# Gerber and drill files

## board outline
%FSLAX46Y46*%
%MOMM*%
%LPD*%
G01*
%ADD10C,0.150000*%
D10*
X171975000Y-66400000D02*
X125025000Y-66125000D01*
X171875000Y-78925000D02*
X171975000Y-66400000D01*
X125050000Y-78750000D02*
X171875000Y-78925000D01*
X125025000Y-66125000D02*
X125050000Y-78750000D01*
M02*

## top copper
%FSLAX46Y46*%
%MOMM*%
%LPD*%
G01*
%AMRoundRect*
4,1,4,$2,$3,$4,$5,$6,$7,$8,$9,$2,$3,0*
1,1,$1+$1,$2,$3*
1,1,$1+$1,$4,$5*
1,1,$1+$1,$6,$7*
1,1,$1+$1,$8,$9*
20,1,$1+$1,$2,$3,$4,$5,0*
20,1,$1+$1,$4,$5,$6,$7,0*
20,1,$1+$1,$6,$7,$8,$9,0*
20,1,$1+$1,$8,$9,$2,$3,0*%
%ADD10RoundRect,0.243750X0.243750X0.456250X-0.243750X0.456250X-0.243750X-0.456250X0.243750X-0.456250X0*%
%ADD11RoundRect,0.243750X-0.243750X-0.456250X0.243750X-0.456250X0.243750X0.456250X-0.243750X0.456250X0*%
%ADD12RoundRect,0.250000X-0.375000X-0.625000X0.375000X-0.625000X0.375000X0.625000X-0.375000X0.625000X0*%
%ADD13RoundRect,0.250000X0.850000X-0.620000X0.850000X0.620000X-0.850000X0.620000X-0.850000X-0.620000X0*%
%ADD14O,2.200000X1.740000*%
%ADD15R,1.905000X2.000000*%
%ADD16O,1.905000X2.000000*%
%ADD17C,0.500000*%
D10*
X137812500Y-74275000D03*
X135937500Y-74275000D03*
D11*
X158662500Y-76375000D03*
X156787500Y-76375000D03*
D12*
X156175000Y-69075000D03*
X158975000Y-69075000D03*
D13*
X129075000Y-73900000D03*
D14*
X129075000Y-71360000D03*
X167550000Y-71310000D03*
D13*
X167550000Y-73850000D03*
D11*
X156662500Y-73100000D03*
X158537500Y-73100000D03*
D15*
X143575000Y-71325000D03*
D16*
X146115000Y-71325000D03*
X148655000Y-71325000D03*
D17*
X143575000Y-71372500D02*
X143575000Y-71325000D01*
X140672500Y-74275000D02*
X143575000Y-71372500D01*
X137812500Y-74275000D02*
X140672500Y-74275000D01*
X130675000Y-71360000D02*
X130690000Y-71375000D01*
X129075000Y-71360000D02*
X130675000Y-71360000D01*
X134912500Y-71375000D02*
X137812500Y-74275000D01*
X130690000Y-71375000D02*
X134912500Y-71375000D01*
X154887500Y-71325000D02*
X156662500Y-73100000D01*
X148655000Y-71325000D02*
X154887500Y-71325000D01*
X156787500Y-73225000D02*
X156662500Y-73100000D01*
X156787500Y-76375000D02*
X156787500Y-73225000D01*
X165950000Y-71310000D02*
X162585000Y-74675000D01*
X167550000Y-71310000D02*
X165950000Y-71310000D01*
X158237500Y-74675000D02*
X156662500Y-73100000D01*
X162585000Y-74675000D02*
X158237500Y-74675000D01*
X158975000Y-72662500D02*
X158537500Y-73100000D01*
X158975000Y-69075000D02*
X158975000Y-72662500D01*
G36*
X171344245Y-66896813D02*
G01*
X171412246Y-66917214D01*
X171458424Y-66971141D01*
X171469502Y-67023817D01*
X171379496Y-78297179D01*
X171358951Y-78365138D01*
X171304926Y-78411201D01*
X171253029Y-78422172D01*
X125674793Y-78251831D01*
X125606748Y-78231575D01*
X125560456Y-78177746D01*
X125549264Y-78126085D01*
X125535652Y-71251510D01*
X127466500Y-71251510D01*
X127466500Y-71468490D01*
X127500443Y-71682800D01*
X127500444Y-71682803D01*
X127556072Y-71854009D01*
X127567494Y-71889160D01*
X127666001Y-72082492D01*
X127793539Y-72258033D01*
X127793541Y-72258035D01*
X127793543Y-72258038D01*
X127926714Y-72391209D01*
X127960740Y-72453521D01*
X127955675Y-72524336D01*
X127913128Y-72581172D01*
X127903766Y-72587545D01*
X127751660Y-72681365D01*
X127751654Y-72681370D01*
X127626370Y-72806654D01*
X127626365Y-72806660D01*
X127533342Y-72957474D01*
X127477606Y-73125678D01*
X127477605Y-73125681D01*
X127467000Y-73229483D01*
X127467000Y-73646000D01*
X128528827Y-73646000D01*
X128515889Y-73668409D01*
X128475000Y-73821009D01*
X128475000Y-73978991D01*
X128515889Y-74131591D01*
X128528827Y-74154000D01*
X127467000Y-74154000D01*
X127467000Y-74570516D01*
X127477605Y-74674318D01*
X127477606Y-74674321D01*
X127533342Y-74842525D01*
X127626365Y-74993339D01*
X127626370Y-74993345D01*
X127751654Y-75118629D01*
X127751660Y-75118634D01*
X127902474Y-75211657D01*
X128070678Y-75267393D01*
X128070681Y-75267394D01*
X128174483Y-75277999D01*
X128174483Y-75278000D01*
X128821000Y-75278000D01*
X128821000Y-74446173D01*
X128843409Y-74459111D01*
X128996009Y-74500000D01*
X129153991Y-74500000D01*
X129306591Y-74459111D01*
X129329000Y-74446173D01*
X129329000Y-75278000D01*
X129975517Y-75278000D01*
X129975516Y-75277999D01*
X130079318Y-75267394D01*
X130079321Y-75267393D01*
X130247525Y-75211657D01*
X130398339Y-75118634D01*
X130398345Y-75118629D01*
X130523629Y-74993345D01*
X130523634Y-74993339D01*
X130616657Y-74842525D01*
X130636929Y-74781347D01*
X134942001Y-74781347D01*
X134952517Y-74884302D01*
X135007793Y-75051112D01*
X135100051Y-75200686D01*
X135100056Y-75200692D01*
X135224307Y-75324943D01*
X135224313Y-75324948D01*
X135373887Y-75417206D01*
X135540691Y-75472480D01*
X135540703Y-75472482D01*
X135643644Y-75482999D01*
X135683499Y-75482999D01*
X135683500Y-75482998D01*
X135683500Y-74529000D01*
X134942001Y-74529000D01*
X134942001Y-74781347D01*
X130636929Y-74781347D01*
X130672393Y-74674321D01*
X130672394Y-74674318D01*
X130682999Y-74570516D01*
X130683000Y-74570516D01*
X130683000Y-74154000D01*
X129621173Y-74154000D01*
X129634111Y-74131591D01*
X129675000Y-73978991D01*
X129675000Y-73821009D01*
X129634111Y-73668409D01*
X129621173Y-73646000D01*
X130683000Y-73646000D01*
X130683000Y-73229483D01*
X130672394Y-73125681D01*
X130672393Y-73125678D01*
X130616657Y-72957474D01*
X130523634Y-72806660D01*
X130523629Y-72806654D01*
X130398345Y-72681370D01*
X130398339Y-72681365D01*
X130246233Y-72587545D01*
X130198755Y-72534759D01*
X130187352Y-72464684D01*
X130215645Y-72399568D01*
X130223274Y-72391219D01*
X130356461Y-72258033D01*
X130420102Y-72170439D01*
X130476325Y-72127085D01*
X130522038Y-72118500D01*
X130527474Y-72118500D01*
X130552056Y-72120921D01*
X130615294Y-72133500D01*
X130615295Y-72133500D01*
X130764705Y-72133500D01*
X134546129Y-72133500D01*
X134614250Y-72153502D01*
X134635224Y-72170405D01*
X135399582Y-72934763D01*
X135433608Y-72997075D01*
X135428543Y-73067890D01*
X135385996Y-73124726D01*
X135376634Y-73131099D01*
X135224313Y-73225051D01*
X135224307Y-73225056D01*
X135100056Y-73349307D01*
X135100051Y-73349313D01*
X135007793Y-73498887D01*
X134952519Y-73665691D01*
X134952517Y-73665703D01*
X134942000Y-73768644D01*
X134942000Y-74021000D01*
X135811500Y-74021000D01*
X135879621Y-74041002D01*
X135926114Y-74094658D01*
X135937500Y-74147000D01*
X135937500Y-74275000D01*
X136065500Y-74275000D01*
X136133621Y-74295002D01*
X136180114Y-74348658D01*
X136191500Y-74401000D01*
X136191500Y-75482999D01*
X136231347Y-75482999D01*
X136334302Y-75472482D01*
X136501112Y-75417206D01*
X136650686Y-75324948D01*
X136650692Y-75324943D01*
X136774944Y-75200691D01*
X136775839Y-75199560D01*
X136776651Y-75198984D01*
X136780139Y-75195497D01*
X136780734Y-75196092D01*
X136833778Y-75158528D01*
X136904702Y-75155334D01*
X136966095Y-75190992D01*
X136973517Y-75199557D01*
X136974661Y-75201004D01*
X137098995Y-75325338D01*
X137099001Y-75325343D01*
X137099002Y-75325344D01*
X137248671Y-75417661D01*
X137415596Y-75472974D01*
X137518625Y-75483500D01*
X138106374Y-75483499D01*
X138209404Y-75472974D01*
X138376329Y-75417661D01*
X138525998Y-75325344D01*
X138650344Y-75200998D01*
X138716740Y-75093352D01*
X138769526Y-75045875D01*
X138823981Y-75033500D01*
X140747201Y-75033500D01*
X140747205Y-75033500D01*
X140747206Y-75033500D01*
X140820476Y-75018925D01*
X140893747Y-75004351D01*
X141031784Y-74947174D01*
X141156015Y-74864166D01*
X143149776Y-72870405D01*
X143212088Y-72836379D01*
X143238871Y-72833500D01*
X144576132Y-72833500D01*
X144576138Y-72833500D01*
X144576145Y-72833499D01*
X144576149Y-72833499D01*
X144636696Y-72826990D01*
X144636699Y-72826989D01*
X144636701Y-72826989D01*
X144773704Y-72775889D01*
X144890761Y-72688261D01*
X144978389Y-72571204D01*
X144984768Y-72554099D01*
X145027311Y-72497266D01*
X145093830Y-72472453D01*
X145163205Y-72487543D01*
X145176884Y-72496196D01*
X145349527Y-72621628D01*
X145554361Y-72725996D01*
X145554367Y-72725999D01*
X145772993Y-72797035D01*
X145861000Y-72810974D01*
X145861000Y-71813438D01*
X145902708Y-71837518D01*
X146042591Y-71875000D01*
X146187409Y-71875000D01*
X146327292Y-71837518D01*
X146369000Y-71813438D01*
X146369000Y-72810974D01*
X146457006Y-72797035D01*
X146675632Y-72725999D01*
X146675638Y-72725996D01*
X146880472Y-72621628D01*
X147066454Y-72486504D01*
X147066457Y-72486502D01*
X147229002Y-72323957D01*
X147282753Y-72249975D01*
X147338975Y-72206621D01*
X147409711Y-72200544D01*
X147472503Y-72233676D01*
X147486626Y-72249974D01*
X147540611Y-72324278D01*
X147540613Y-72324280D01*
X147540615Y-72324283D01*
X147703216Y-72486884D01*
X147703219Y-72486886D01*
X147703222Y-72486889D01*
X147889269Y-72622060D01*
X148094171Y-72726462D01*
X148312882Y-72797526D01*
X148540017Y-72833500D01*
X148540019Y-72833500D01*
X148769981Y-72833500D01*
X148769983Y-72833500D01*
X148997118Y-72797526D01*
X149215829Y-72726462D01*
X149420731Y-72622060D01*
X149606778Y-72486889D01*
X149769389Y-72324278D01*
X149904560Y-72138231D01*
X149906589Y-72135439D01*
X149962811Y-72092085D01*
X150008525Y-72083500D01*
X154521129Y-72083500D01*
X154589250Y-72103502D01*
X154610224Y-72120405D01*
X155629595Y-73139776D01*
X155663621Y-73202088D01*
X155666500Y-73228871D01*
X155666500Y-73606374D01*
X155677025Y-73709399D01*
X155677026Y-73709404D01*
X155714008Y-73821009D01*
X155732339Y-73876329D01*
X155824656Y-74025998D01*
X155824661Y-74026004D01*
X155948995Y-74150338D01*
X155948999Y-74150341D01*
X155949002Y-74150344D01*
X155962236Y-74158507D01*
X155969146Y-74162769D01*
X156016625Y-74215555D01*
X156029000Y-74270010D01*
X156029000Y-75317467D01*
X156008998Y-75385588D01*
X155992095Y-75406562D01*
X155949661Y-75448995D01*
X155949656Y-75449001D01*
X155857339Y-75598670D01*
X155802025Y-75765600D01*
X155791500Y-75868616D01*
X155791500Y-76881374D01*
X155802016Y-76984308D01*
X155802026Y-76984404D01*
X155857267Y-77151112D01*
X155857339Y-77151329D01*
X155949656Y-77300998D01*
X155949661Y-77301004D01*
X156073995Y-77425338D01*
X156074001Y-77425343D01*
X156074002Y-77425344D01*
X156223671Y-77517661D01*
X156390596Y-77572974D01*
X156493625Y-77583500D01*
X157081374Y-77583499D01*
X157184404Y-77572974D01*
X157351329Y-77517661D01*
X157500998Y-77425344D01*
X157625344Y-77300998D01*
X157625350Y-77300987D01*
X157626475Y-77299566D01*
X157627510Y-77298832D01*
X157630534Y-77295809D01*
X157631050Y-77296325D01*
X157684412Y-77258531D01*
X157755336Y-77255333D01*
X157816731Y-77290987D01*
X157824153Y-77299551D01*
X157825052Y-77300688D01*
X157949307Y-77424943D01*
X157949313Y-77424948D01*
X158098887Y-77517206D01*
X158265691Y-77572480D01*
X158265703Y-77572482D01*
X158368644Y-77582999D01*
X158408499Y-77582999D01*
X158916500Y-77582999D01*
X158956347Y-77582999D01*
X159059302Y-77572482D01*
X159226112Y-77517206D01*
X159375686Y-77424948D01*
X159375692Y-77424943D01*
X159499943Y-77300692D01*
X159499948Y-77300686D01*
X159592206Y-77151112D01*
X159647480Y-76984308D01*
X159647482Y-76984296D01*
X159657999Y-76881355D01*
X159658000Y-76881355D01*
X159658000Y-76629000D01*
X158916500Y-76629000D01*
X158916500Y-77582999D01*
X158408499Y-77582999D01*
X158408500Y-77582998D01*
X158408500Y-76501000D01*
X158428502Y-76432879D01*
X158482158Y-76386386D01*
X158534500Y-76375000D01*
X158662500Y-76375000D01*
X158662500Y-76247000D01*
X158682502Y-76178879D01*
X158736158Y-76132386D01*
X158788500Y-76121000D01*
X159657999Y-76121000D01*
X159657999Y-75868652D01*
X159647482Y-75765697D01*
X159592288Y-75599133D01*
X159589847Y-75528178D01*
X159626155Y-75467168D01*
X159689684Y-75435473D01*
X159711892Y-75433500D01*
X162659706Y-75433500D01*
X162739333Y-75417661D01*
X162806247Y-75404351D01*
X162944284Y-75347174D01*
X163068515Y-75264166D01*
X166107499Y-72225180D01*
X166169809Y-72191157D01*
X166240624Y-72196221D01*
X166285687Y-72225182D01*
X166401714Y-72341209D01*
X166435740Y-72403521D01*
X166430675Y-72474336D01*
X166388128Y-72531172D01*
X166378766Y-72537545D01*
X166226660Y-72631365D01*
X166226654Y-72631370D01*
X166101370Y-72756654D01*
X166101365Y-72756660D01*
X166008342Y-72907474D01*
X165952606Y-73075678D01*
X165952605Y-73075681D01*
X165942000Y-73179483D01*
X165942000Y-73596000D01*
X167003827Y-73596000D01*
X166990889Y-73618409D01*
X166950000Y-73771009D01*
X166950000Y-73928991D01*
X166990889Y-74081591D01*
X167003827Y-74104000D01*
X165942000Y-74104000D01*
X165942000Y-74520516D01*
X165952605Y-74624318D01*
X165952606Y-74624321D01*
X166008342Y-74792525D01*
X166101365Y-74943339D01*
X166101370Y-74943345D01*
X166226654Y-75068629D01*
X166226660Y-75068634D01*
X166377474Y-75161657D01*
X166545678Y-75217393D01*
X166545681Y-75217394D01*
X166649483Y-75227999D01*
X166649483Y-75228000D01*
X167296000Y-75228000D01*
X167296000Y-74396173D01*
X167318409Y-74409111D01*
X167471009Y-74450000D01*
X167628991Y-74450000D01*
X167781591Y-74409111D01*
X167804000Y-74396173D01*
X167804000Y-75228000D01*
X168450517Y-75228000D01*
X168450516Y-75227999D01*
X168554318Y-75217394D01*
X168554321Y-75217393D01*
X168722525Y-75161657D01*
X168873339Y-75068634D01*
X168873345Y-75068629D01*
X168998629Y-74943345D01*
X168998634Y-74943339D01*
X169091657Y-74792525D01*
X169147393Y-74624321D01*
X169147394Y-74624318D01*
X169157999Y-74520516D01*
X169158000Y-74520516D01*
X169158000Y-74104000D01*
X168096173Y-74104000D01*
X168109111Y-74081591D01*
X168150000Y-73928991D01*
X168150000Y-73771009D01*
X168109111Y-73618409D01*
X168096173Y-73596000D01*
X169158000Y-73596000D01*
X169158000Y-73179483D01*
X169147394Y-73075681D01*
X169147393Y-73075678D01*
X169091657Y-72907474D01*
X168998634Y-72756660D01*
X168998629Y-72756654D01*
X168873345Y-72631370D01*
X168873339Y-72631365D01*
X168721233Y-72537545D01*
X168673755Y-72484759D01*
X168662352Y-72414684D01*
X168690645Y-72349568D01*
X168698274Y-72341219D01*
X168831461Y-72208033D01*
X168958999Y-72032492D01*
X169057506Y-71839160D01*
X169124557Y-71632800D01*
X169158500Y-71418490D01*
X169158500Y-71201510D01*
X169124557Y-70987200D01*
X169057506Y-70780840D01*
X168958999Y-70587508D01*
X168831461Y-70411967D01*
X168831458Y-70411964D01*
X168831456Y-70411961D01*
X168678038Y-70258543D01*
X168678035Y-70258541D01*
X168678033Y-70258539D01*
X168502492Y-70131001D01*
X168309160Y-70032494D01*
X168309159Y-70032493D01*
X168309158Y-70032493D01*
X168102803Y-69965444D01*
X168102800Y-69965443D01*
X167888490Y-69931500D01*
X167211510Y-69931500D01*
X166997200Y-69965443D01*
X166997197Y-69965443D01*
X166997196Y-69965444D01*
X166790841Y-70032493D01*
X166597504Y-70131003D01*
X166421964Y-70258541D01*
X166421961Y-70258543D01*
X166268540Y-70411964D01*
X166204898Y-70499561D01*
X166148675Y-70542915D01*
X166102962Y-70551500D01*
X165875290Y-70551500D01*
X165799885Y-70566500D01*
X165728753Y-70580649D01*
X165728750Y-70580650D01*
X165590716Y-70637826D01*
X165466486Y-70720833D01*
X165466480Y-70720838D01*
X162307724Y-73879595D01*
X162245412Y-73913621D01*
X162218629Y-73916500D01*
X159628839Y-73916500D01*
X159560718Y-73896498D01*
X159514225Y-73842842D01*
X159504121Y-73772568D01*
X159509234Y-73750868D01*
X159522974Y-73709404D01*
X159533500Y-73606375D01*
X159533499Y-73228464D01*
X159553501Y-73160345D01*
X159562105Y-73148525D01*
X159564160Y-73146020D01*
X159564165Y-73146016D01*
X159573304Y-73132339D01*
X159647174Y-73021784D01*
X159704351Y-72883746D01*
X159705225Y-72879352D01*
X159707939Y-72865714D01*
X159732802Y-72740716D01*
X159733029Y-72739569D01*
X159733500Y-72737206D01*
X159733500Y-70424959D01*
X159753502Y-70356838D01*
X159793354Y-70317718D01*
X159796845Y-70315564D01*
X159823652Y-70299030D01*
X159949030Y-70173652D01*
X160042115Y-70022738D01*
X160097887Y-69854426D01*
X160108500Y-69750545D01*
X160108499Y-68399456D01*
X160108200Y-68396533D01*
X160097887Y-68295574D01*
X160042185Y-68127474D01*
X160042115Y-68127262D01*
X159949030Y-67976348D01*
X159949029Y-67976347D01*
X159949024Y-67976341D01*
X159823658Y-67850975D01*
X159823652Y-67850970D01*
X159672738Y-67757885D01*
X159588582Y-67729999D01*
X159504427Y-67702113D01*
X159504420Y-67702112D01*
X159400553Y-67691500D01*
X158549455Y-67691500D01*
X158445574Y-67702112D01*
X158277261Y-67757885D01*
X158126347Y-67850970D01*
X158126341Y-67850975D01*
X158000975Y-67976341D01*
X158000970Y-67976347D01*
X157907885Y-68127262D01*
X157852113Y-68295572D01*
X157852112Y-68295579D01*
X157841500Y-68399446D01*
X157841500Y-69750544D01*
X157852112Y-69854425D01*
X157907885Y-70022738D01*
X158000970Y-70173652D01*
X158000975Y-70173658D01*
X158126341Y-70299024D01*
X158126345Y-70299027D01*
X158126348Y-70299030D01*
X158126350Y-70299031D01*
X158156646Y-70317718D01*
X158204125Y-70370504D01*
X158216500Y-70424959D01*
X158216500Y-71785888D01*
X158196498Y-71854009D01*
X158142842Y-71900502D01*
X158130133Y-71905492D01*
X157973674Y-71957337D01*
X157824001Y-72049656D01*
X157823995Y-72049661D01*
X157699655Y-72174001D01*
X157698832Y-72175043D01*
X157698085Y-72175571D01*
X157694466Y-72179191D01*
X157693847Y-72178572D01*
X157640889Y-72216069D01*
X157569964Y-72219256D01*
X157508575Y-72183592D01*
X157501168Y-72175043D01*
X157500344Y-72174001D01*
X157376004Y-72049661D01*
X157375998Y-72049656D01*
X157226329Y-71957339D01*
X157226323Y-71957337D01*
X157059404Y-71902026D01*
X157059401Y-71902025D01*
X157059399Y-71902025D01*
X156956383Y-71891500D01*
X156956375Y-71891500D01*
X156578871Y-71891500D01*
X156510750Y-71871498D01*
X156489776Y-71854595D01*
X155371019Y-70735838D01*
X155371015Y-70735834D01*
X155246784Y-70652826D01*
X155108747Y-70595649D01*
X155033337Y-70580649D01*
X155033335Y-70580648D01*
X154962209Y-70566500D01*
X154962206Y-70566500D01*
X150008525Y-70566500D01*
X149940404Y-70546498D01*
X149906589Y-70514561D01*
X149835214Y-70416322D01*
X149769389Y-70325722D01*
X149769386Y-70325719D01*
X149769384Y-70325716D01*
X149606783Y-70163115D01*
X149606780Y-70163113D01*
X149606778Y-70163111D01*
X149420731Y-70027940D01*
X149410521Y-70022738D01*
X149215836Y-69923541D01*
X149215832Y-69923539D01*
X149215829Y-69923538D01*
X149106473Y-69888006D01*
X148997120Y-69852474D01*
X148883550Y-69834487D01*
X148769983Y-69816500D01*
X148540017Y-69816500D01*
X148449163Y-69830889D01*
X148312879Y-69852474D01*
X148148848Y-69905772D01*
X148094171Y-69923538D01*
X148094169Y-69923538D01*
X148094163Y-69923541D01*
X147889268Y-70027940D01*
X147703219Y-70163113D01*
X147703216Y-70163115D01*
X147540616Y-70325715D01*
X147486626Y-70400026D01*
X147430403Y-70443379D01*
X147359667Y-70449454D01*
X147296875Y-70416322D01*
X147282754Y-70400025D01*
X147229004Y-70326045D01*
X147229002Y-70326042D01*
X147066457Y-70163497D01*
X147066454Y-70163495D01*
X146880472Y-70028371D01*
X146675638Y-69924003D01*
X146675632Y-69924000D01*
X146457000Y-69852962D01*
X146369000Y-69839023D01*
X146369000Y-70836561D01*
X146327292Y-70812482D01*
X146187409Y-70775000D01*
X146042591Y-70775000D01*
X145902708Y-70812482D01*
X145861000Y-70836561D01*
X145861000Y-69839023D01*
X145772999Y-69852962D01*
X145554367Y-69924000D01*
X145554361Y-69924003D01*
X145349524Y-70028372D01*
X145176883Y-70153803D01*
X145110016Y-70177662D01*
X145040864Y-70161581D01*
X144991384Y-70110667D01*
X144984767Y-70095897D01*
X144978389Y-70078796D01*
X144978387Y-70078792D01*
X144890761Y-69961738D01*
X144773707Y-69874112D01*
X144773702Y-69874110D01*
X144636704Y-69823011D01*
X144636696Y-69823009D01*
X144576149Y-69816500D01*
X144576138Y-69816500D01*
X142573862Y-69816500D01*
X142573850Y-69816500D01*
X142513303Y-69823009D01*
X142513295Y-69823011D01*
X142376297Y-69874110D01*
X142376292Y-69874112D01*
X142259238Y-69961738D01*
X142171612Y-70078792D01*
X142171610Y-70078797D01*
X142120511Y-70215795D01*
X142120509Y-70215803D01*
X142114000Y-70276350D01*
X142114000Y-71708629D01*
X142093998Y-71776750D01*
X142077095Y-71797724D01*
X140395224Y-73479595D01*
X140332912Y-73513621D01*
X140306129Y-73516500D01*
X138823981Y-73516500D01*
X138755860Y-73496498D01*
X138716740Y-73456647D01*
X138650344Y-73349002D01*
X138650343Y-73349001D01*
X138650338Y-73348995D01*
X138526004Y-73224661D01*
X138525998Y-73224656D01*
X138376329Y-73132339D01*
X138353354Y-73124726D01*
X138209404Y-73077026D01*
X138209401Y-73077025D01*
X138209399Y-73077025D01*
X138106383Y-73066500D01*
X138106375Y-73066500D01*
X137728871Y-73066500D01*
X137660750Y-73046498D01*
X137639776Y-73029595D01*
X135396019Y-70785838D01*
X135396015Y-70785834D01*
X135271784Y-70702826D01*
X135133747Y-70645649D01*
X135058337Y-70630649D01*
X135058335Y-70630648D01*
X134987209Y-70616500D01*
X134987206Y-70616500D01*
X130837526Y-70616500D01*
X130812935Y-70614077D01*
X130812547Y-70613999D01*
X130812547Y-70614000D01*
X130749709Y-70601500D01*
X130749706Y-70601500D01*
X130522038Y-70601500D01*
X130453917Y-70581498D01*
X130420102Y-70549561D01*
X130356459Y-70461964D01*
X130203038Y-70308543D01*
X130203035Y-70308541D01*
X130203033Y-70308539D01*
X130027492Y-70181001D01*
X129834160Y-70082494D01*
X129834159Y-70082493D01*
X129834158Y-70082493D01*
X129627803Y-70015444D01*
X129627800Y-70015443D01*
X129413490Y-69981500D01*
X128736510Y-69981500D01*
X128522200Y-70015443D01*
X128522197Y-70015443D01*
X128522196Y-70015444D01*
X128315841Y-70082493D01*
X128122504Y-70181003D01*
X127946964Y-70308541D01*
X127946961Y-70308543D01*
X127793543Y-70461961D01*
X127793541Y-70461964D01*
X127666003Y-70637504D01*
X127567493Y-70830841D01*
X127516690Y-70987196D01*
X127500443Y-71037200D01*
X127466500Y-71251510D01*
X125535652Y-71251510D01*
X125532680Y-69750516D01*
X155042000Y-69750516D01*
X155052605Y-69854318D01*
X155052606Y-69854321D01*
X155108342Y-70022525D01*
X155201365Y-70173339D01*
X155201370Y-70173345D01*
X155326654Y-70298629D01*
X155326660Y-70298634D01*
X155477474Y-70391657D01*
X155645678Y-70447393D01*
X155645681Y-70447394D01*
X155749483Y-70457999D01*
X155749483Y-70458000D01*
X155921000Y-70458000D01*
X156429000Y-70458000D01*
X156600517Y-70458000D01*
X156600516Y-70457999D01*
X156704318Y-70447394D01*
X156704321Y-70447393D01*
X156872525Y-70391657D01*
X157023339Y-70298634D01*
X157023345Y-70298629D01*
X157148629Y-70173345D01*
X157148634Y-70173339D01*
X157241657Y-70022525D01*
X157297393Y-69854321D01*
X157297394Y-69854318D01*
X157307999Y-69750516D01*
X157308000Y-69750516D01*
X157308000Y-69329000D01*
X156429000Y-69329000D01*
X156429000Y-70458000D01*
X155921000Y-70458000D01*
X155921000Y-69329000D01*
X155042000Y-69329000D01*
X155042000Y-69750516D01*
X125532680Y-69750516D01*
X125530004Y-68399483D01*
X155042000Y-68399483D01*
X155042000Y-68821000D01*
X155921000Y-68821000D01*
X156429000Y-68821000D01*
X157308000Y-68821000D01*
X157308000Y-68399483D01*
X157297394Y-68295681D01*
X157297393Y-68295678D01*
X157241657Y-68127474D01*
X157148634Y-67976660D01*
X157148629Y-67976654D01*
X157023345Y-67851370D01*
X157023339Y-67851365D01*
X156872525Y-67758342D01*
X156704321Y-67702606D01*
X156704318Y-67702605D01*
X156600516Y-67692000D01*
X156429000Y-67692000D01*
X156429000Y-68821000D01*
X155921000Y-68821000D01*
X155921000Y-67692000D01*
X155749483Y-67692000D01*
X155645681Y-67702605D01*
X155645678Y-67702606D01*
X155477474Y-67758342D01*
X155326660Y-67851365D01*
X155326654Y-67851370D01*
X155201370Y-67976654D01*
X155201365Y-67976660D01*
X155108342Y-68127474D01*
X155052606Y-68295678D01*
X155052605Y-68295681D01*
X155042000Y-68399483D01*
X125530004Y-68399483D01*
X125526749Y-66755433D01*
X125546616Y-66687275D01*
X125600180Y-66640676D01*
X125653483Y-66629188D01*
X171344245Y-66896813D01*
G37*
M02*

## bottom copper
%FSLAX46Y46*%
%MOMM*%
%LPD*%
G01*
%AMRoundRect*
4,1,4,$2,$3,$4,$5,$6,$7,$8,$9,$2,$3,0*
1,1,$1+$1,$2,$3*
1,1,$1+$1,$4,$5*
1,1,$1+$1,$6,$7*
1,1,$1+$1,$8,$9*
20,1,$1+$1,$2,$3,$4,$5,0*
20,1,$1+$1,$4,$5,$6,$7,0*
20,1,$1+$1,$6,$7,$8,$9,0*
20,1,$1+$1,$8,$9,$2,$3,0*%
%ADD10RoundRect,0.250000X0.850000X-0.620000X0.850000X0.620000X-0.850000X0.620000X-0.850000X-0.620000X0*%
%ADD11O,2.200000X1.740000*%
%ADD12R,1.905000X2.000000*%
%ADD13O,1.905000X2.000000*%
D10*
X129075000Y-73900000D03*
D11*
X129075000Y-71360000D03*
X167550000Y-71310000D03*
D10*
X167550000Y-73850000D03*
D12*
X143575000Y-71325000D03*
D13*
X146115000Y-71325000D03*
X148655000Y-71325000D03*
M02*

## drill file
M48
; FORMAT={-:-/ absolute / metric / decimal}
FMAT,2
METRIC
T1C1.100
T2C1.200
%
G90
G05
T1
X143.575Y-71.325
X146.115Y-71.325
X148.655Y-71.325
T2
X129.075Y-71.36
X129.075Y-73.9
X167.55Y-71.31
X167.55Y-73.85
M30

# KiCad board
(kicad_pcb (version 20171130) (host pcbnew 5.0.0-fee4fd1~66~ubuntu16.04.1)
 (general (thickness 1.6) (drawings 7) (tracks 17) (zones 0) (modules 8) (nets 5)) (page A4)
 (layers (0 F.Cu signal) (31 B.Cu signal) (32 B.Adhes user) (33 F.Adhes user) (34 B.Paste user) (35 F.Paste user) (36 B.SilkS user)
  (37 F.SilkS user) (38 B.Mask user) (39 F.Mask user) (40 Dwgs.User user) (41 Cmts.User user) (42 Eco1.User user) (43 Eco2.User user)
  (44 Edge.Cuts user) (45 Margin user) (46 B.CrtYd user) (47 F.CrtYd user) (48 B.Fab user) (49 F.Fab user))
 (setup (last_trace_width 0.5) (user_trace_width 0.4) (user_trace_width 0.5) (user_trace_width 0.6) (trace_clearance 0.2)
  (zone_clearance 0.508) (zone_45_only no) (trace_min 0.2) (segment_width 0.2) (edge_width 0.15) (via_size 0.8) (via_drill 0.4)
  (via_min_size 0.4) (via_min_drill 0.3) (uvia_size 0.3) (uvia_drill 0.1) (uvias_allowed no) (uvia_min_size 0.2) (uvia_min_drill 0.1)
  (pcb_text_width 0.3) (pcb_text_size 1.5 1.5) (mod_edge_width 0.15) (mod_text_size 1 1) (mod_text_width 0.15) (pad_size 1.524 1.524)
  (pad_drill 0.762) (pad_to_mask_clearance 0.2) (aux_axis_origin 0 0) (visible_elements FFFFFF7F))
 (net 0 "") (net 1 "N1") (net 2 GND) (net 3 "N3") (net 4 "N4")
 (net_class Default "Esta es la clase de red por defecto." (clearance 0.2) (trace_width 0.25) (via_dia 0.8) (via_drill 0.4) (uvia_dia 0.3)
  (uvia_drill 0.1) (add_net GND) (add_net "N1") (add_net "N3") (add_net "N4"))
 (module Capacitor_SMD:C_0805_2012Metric (layer F.Cu) (at 136.875 74.275 180)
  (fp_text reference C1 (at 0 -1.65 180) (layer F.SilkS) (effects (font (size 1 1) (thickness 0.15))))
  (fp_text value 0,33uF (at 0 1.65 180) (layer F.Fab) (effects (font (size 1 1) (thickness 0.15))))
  (pad 1 smd roundrect (at -0.9375 0 180) (size 0.975 1.4) (layers F.Cu F.Paste F.Mask) (roundrect_rratio 0.25) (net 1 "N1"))
  (pad 2 smd roundrect (at 0.9375 0 180) (size 0.975 1.4) (layers F.Cu F.Paste F.Mask) (roundrect_rratio 0.25) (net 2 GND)))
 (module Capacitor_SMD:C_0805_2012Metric (layer F.Cu) (at 157.725 76.375)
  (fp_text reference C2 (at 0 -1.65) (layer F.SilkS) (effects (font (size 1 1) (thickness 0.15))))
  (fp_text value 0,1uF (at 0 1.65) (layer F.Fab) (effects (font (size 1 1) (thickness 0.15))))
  (pad 2 smd roundrect (at 0.9375 0) (size 0.975 1.4) (layers F.Cu F.Paste F.Mask) (roundrect_rratio 0.25) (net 2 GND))
  (pad 1 smd roundrect (at -0.9375 0) (size 0.975 1.4) (layers F.Cu F.Paste F.Mask) (roundrect_rratio 0.25) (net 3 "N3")))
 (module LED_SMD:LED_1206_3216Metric (layer F.Cu) (at 157.575 69.075)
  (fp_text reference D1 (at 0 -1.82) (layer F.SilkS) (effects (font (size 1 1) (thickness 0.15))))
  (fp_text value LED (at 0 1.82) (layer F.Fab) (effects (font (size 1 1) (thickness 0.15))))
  (pad 1 smd roundrect (at -1.4 0) (size 1.25 1.75) (layers F.Cu F.Paste F.Mask) (roundrect_rratio 0.2) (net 2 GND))
  (pad 2 smd roundrect (at 1.4 0) (size 1.25 1.75) (layers F.Cu F.Paste F.Mask) (roundrect_rratio 0.2) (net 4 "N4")))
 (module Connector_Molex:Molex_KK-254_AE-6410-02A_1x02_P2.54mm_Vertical (layer F.Cu) (at 129.075 73.9 90)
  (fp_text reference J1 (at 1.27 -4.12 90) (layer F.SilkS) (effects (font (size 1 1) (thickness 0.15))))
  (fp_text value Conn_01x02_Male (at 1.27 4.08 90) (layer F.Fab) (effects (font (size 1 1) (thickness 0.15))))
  (pad 1 thru_hole roundrect (at 0 0 90) (size 1.74 2.2) (drill 1.2) (layers *.Cu *.Mask) (roundrect_rratio 0.143678) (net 2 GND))
  (pad 2 thru_hole oval (at 2.54 0 90) (size 1.74 2.2) (drill 1.2) (layers *.Cu *.Mask) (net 1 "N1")))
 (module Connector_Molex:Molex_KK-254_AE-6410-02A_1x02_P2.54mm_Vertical (layer F.Cu) (at 167.55 73.85 90)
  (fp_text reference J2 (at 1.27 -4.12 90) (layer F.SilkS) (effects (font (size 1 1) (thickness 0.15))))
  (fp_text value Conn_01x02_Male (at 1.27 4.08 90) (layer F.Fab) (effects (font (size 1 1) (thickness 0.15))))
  (pad 2 thru_hole oval (at 2.54 0 90) (size 1.74 2.2) (drill 1.2) (layers *.Cu *.Mask) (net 3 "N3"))
  (pad 1 thru_hole roundrect (at 0 0 90) (size 1.74 2.2) (drill 1.2) (layers *.Cu *.Mask) (roundrect_rratio 0.143678) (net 2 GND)))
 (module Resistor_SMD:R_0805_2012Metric (layer F.Cu) (at 157.6 73.1)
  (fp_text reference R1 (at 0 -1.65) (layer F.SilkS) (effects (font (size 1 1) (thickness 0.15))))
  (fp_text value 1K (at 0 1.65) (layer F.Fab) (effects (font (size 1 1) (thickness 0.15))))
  (pad 1 smd roundrect (at -0.9375 0) (size 0.975 1.4) (layers F.Cu F.Paste F.Mask) (roundrect_rratio 0.25) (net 3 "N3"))
  (pad 2 smd roundrect (at 0.9375 0) (size 0.975 1.4) (layers F.Cu F.Paste F.Mask) (roundrect_rratio 0.25) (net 4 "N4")))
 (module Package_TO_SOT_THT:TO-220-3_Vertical (layer F.Cu) (at 143.575 71.325)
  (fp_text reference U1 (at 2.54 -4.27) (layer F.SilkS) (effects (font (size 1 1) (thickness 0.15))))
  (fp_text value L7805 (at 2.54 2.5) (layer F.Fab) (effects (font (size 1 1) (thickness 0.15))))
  (pad 1 thru_hole rect (at 0 0) (size 1.905 2) (drill 1.1) (layers *.Cu *.Mask) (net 1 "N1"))
  (pad 2 thru_hole oval (at 2.54 0) (size 1.905 2) (drill 1.1) (layers *.Cu *.Mask) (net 2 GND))
  (pad 3 thru_hole oval (at 5.08 0) (size 1.905 2) (drill 1.1) (layers *.Cu *.Mask) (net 3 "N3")))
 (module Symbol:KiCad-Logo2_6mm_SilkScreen (layer B.Cu) (at 157.63 71.98 180)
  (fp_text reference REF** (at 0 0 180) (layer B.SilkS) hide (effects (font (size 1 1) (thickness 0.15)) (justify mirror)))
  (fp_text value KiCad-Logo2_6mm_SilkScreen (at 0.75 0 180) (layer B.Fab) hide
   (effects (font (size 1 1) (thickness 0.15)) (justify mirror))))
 (gr_line (start 171.975 66.4) (end 125.025 66.125) (layer Edge.Cuts) (width 0.15))
 (gr_line (start 171.875 78.925) (end 171.975 66.4) (layer Edge.Cuts) (width 0.15))
 (gr_line (start 125.05 78.75) (end 171.875 78.925) (layer Edge.Cuts) (width 0.15))
 (gr_line (start 125.025 66.125) (end 125.05 78.75) (layer Edge.Cuts) (width 0.15))
 (segment (start 143.575 71.3725) (end 143.575 71.325) (width 0.5) (layer F.Cu) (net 1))
 (segment (start 140.6725 74.275) (end 143.575 71.3725) (width 0.5) (layer F.Cu) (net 1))
 (segment (start 137.8125 74.275) (end 140.6725 74.275) (width 0.5) (layer F.Cu) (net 1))
 (segment (start 130.675 71.36) (end 130.69 71.375) (width 0.5) (layer F.Cu) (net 1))
 (segment (start 129.075 71.36) (end 130.675 71.36) (width 0.5) (layer F.Cu) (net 1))
 (segment (start 134.9125 71.375) (end 137.8125 74.275) (width 0.5) (layer F.Cu) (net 1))
 (segment (start 130.69 71.375) (end 134.9125 71.375) (width 0.5) (layer F.Cu) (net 1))
 (segment (start 154.8875 71.325) (end 156.6625 73.1) (width 0.5) (layer F.Cu) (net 3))
 (segment (start 148.655 71.325) (end 154.8875 71.325) (width 0.5) (layer F.Cu) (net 3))
 (segment (start 156.7875 73.225) (end 156.6625 73.1) (width 0.5) (layer F.Cu) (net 3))
 (segment (start 156.7875 76.375) (end 156.7875 73.225) (width 0.5) (layer F.Cu) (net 3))
 (segment (start 165.95 71.31) (end 162.585 74.675) (width 0.5) (layer F.Cu) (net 3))
 (segment (start 167.55 71.31) (end 165.95 71.31) (width 0.5) (layer F.Cu) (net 3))
 (segment (start 158.2375 74.675) (end 156.6625 73.1) (width 0.5) (layer F.Cu) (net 3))
 (segment (start 162.585 74.675) (end 158.2375 74.675) (width 0.5) (layer F.Cu) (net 3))
 (segment (start 158.975 72.6625) (end 158.5375 73.1) (width 0.5) (layer F.Cu) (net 4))
 (segment (start 158.975 69.075) (end 158.975 72.6625) (width 0.5) (layer F.Cu) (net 4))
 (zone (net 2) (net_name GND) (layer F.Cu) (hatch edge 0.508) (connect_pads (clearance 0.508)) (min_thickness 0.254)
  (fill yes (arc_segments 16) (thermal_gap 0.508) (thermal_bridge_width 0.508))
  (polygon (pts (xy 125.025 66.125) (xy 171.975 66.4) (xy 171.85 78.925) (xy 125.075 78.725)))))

